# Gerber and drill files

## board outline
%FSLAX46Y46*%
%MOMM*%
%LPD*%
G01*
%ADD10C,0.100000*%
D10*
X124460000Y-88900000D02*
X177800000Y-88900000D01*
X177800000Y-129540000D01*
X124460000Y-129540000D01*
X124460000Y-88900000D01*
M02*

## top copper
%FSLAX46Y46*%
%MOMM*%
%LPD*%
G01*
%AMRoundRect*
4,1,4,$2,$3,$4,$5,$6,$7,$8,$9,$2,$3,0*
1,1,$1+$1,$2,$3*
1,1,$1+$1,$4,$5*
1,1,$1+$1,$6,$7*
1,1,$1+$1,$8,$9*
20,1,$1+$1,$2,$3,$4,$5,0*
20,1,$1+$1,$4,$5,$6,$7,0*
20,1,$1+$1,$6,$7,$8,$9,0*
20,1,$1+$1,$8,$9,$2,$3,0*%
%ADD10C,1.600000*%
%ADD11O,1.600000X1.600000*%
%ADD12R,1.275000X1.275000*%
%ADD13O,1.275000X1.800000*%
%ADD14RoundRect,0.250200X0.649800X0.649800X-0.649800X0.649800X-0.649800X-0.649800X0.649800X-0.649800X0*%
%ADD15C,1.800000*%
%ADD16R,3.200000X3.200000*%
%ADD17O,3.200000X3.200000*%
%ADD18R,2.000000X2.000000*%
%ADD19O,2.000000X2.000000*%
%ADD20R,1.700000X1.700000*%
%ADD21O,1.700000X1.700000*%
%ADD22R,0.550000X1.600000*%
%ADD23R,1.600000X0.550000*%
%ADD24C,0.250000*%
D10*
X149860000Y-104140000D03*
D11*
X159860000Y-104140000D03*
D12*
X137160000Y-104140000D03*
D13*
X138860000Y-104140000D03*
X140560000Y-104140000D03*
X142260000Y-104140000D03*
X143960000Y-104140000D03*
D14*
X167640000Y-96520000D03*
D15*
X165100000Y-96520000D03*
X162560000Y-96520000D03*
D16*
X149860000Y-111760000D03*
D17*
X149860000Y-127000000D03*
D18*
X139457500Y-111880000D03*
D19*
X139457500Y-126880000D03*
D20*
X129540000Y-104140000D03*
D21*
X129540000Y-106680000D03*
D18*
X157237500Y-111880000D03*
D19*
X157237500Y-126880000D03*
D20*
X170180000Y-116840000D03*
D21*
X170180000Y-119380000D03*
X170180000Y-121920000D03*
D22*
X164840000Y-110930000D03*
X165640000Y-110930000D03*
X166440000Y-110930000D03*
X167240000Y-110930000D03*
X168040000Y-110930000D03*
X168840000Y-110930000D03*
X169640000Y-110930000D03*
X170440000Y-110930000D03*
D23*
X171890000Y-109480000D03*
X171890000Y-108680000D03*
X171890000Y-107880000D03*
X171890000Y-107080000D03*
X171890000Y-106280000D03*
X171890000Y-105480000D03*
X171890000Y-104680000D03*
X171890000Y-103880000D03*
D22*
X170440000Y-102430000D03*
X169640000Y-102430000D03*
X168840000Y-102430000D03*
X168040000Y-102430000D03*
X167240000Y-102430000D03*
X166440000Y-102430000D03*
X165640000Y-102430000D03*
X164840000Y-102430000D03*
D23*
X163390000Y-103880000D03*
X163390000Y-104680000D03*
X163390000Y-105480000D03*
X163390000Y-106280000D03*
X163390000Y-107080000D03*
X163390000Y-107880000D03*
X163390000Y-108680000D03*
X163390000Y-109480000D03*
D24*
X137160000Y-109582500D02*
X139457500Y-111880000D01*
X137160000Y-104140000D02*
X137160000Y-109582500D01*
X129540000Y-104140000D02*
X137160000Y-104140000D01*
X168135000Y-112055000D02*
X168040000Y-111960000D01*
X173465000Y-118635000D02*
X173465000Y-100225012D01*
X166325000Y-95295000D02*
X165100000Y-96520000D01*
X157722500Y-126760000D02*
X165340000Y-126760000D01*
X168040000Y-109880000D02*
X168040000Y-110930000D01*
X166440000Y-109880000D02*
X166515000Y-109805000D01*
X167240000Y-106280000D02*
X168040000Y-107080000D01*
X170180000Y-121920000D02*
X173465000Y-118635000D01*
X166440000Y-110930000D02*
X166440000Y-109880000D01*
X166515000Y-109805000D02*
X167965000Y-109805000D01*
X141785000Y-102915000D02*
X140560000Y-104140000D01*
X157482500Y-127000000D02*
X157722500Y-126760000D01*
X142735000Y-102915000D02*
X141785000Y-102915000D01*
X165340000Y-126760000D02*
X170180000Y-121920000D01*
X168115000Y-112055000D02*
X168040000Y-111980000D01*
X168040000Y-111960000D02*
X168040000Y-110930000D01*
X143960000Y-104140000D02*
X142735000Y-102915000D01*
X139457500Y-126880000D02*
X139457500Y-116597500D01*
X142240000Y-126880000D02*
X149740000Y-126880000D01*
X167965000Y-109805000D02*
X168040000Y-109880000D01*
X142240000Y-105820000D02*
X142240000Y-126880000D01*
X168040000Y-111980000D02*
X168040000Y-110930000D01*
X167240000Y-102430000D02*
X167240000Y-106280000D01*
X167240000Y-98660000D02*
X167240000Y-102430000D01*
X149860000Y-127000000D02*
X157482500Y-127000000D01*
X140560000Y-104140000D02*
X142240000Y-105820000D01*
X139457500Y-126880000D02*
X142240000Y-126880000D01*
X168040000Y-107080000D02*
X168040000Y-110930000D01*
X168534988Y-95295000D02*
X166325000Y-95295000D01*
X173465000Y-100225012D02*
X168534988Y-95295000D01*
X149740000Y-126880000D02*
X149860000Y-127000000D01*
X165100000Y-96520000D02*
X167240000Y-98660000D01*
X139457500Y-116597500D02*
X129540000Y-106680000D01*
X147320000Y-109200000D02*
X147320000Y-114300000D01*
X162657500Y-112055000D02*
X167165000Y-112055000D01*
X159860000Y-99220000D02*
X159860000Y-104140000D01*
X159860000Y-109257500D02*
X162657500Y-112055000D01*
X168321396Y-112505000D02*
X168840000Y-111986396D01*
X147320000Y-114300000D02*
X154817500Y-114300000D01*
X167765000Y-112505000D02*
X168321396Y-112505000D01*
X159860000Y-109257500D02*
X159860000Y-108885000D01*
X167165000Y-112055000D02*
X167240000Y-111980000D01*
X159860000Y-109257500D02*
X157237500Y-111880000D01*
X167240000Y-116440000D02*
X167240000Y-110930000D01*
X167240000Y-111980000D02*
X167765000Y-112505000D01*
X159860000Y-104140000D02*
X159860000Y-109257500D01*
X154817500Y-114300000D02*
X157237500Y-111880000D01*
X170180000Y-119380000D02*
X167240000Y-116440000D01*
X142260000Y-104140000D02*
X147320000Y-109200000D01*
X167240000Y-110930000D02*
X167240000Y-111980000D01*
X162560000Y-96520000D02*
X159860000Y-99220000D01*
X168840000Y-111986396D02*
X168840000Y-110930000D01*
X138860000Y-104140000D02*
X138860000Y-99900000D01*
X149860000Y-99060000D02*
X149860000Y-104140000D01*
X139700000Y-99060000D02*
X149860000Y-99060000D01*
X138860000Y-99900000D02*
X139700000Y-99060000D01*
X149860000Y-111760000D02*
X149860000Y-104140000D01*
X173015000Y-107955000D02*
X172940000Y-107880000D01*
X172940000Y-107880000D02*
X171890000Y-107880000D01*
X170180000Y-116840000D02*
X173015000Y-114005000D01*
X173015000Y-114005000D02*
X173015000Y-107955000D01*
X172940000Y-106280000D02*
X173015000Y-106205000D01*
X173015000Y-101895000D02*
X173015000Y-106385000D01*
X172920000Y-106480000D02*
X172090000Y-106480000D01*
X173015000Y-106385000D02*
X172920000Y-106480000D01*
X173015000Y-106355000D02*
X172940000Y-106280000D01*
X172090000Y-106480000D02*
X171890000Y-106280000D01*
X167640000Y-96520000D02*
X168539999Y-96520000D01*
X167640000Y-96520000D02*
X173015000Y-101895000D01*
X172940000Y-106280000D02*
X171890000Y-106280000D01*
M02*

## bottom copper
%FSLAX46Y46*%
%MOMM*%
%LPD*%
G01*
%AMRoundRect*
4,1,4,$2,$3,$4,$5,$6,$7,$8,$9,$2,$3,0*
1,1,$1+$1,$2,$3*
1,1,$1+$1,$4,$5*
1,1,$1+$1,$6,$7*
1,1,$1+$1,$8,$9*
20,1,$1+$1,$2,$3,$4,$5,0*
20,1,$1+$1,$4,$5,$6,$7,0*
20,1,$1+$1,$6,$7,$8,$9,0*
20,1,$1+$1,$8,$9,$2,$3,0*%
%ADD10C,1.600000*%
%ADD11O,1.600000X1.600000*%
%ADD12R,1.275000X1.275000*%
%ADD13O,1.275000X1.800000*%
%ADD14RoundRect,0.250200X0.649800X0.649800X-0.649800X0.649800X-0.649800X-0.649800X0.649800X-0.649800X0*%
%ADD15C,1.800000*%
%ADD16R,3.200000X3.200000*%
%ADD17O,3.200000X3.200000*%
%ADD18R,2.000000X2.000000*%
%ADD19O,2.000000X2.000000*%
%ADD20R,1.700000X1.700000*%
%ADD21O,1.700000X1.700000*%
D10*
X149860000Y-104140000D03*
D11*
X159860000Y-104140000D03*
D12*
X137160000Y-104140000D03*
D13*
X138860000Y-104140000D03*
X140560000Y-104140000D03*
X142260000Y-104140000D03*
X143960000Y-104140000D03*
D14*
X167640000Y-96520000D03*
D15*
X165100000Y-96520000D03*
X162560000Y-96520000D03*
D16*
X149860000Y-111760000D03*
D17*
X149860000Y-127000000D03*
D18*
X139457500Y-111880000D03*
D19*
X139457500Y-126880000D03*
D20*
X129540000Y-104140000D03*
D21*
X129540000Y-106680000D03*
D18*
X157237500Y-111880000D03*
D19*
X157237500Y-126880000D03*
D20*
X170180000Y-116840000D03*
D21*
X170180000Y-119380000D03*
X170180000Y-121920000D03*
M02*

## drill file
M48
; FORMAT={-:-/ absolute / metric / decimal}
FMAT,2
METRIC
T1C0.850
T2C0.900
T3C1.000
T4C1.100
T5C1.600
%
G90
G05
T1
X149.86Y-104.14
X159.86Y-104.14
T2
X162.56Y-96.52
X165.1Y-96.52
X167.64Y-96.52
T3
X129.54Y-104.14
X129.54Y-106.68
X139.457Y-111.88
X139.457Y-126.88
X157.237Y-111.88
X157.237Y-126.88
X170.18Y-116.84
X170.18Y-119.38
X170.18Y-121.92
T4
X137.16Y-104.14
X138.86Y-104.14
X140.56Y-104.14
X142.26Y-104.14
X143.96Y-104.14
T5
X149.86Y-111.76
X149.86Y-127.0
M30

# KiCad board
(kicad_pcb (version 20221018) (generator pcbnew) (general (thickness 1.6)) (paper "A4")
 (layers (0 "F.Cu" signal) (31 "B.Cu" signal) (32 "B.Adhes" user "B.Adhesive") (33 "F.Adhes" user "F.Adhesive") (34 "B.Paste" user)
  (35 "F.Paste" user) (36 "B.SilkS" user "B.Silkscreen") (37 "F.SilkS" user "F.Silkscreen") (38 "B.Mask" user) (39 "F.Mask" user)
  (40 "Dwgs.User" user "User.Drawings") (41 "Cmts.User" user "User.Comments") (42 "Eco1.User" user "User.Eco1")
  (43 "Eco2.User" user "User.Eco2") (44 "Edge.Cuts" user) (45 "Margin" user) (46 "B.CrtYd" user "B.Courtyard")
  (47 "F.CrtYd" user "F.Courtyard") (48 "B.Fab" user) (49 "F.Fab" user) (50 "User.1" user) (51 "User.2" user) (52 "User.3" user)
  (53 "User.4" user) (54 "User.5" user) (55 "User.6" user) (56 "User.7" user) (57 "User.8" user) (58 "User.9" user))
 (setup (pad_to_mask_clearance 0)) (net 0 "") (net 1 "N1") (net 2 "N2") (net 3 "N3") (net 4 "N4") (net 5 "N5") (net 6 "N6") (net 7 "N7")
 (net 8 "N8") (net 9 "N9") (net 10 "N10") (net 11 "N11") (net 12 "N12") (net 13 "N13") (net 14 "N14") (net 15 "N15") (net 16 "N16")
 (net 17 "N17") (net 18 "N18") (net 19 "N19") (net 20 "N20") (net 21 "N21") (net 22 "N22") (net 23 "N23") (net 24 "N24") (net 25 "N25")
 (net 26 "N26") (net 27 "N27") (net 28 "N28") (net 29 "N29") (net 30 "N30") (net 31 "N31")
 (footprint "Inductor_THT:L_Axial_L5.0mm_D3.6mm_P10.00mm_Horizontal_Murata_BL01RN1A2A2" (layer "F.Cu") (at 149.86 104.14)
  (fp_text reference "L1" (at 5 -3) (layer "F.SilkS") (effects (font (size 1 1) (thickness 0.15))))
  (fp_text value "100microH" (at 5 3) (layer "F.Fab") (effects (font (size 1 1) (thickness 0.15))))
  (pad "1" thru_hole circle (at 0 0) (size 1.6 1.6) (drill 0.85) (layers "*.Cu" "*.Mask") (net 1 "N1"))
  (pad "2" thru_hole oval (at 10 0) (size 1.6 1.6) (drill 0.85) (layers "*.Cu" "*.Mask") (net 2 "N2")))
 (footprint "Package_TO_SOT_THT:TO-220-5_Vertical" (layer "F.Cu") (at 137.16 104.14)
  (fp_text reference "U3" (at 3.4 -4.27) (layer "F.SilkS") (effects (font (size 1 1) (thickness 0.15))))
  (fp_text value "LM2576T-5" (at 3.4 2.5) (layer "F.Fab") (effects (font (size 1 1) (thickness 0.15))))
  (pad "1" thru_hole rect (at 0 0) (size 1.275 1.275) (drill 1.1) (layers "*.Cu" "*.Mask") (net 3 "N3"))
  (pad "2" thru_hole oval (at 1.7 0) (size 1.275 1.8) (drill 1.1) (layers "*.Cu" "*.Mask") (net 1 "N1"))
  (pad "3" thru_hole oval (at 3.4 0) (size 1.275 1.8) (drill 1.1) (layers "*.Cu" "*.Mask") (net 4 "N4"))
  (pad "4" thru_hole oval (at 5.1 0) (size 1.275 1.8) (drill 1.1) (layers "*.Cu" "*.Mask") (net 2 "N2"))
  (pad "5" thru_hole oval (at 6.8 0) (size 1.275 1.8) (drill 1.1) (layers "*.Cu" "*.Mask") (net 4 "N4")))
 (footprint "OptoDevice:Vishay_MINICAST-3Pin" (layer "F.Cu") (at 167.64 96.52 180)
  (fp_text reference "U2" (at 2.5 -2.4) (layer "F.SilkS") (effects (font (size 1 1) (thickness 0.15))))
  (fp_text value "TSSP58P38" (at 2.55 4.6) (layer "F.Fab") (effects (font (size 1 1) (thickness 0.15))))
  (pad "1" thru_hole roundrect (at 0 0 180) (size 1.8 1.8) (drill 0.9) (layers "*.Cu" "*.Mask") (roundrect_rratio 0.139) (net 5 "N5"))
  (pad "2" thru_hole circle (at 2.54 0 180) (size 1.8 1.8) (drill 0.9) (layers "*.Cu" "*.Mask") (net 4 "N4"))
  (pad "3" thru_hole circle (at 5.08 0 180) (size 1.8 1.8) (drill 0.9) (layers "*.Cu" "*.Mask") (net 2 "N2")))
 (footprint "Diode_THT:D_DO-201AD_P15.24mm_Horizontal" (layer "F.Cu") (at 149.86 111.76 -90)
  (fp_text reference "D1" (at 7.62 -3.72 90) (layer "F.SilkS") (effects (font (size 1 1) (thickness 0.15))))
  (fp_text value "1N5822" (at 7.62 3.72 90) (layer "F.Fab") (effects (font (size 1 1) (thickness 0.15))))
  (pad "1" thru_hole rect (at 0 0 270) (size 3.2 3.2) (drill 1.6) (layers "*.Cu" "*.Mask") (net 1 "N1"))
  (pad "2" thru_hole oval (at 15.24 0 270) (size 3.2 3.2) (drill 1.6) (layers "*.Cu" "*.Mask") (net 4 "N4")))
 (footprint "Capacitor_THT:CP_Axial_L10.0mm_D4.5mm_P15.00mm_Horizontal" (layer "F.Cu") (at 139.4575 111.88 -90)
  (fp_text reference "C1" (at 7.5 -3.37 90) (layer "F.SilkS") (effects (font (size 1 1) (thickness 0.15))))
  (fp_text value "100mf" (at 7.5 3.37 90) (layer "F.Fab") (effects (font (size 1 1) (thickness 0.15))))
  (pad "1" thru_hole rect (at 0 0 270) (size 2 2) (drill 1) (layers "*.Cu" "*.Mask") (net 3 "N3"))
  (pad "2" thru_hole oval (at 15 0 270) (size 2 2) (drill 1) (layers "*.Cu" "*.Mask") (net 4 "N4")))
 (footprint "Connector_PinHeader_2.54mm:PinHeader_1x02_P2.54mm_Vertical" (layer "F.Cu") (at 129.54 104.14)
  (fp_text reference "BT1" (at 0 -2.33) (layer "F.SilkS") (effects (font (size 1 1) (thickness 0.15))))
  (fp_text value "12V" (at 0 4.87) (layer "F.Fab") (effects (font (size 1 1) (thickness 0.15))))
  (pad "1" thru_hole rect (at 0 0) (size 1.7 1.7) (drill 1) (layers "*.Cu" "*.Mask") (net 3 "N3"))
  (pad "2" thru_hole oval (at 0 2.54) (size 1.7 1.7) (drill 1) (layers "*.Cu" "*.Mask") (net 4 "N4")))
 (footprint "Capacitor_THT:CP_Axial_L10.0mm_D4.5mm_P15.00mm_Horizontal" (layer "F.Cu") (at 157.2375 111.88 -90)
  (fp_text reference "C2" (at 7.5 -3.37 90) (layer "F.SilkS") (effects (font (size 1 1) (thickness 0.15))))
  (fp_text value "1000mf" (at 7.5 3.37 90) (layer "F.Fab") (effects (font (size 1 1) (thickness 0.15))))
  (pad "1" thru_hole rect (at 0 0 270) (size 2 2) (drill 1) (layers "*.Cu" "*.Mask") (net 2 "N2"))
  (pad "2" thru_hole oval (at 15 0 270) (size 2 2) (drill 1) (layers "*.Cu" "*.Mask") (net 4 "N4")))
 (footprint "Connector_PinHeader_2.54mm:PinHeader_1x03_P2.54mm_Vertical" (layer "F.Cu") (at 170.18 116.84)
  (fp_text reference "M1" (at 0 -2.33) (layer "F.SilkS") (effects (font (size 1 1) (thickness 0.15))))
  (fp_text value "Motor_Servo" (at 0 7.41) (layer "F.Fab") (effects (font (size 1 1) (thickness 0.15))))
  (pad "1" thru_hole rect (at 0 0) (size 1.7 1.7) (drill 1) (layers "*.Cu" "*.Mask") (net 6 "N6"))
  (pad "2" thru_hole oval (at 0 2.54) (size 1.7 1.7) (drill 1) (layers "*.Cu" "*.Mask") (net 2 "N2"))
  (pad "3" thru_hole oval (at 0 5.08) (size 1.7 1.7) (drill 1) (layers "*.Cu" "*.Mask") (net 4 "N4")))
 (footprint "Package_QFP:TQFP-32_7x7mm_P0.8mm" (layer "F.Cu") (at 167.64 106.68 90)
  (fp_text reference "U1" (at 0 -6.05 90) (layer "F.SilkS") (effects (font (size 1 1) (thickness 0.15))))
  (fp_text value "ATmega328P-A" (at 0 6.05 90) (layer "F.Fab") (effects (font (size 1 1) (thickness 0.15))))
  (pad "1" smd rect (at -4.25 -2.8 90) (size 1.6 0.55) (layers "F.Cu" "F.Paste" "F.Mask") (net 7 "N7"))
  (pad "2" smd rect (at -4.25 -2 90) (size 1.6 0.55) (layers "F.Cu" "F.Paste" "F.Mask") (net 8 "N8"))
  (pad "3" smd rect (at -4.25 -1.2 90) (size 1.6 0.55) (layers "F.Cu" "F.Paste" "F.Mask") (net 4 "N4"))
  (pad "4" smd rect (at -4.25 -0.4 90) (size 1.6 0.55) (layers "F.Cu" "F.Paste" "F.Mask") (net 2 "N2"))
  (pad "5" smd rect (at -4.25 0.4 90) (size 1.6 0.55) (layers "F.Cu" "F.Paste" "F.Mask") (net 4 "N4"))
  (pad "6" smd rect (at -4.25 1.2 90) (size 1.6 0.55) (layers "F.Cu" "F.Paste" "F.Mask") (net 2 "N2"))
  (pad "7" smd rect (at -4.25 2 90) (size 1.6 0.55) (layers "F.Cu" "F.Paste" "F.Mask") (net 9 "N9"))
  (pad "8" smd rect (at -4.25 2.8 90) (size 1.6 0.55) (layers "F.Cu" "F.Paste" "F.Mask") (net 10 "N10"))
  (pad "9" smd rect (at -2.8 4.25 180) (size 1.6 0.55) (layers "F.Cu" "F.Paste" "F.Mask") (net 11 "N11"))
  (pad "10" smd rect (at -2 4.25 180) (size 1.6 0.55) (layers "F.Cu" "F.Paste" "F.Mask") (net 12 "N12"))
  (pad "11" smd rect (at -1.2 4.25 180) (size 1.6 0.55) (layers "F.Cu" "F.Paste" "F.Mask") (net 6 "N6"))
  (pad "12" smd rect (at -0.4 4.25 180) (size 1.6 0.55) (layers "F.Cu" "F.Paste" "F.Mask") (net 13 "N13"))
  (pad "13" smd rect (at 0.4 4.25 180) (size 1.6 0.55) (layers "F.Cu" "F.Paste" "F.Mask") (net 5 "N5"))
  (pad "14" smd rect (at 1.2 4.25 180) (size 1.6 0.55) (layers "F.Cu" "F.Paste" "F.Mask") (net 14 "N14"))
  (pad "15" smd rect (at 2 4.25 180) (size 1.6 0.55) (layers "F.Cu" "F.Paste" "F.Mask") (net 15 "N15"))
  (pad "16" smd rect (at 2.8 4.25 180) (size 1.6 0.55) (layers "F.Cu" "F.Paste" "F.Mask") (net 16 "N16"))
  (pad "17" smd rect (at 4.25 2.8 90) (size 1.6 0.55) (layers "F.Cu" "F.Paste" "F.Mask") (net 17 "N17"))
  (pad "18" smd rect (at 4.25 2 90) (size 1.6 0.55) (layers "F.Cu" "F.Paste" "F.Mask") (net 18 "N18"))
  (pad "19" smd rect (at 4.25 1.2 90) (size 1.6 0.55) (layers "F.Cu" "F.Paste" "F.Mask") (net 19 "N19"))
  (pad "20" smd rect (at 4.25 0.4 90) (size 1.6 0.55) (layers "F.Cu" "F.Paste" "F.Mask") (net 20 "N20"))
  (pad "21" smd rect (at 4.25 -0.4 90) (size 1.6 0.55) (layers "F.Cu" "F.Paste" "F.Mask") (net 4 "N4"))
  (pad "22" smd rect (at 4.25 -1.2 90) (size 1.6 0.55) (layers "F.Cu" "F.Paste" "F.Mask") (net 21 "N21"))
  (pad "23" smd rect (at 4.25 -2 90) (size 1.6 0.55) (layers "F.Cu" "F.Paste" "F.Mask") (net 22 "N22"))
  (pad "24" smd rect (at 4.25 -2.8 90) (size 1.6 0.55) (layers "F.Cu" "F.Paste" "F.Mask") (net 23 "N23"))
  (pad "25" smd rect (at 2.8 -4.25 180) (size 1.6 0.55) (layers "F.Cu" "F.Paste" "F.Mask") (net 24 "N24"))
  (pad "26" smd rect (at 2 -4.25 180) (size 1.6 0.55) (layers "F.Cu" "F.Paste" "F.Mask") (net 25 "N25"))
  (pad "27" smd rect (at 1.2 -4.25 180) (size 1.6 0.55) (layers "F.Cu" "F.Paste" "F.Mask") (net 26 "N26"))
  (pad "28" smd rect (at 0.4 -4.25 180) (size 1.6 0.55) (layers "F.Cu" "F.Paste" "F.Mask") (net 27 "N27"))
  (pad "29" smd rect (at -0.4 -4.25 180) (size 1.6 0.55) (layers "F.Cu" "F.Paste" "F.Mask") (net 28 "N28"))
  (pad "30" smd rect (at -1.2 -4.25 180) (size 1.6 0.55) (layers "F.Cu" "F.Paste" "F.Mask") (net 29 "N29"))
  (pad "31" smd rect (at -2 -4.25 180) (size 1.6 0.55) (layers "F.Cu" "F.Paste" "F.Mask") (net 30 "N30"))
  (pad "32" smd rect (at -2.8 -4.25 180) (size 1.6 0.55) (layers "F.Cu" "F.Paste" "F.Mask") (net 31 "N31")))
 (gr_rect (start 124.46 88.9) (end 177.8 129.54) (stroke (width 0.1) (type default)) (fill none) (layer "Edge.Cuts"))
 (segment (start 137.16 109.5825) (end 139.4575 111.88) (width 0.25) (layer "F.Cu") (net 3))
 (segment (start 137.16 104.14) (end 137.16 109.5825) (width 0.25) (layer "F.Cu") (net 3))
 (segment (start 129.54 104.14) (end 137.16 104.14) (width 0.25) (layer "F.Cu") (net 3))
 (segment (start 168.135 112.055) (end 168.04 111.96) (width 0.25) (layer "F.Cu") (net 4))
 (segment (start 173.465 118.635) (end 173.465 100.225012) (width 0.25) (layer "F.Cu") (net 4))
 (segment (start 166.325 95.295) (end 165.1 96.52) (width 0.25) (layer "F.Cu") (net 4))
 (segment (start 157.7225 126.76) (end 165.34 126.76) (width 0.25) (layer "F.Cu") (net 4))
 (segment (start 168.04 109.88) (end 168.04 110.93) (width 0.25) (layer "F.Cu") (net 4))
 (segment (start 166.44 109.88) (end 166.515 109.805) (width 0.25) (layer "F.Cu") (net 4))
 (segment (start 167.24 106.28) (end 168.04 107.08) (width 0.25) (layer "F.Cu") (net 4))
 (segment (start 170.18 121.92) (end 173.465 118.635) (width 0.25) (layer "F.Cu") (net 4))
 (segment (start 166.44 110.93) (end 166.44 109.88) (width 0.25) (layer "F.Cu") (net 4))
 (segment (start 166.515 109.805) (end 167.965 109.805) (width 0.25) (layer "F.Cu") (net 4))
 (segment (start 141.785 102.915) (end 140.56 104.14) (width 0.25) (layer "F.Cu") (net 4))
 (segment (start 157.4825 127) (end 157.7225 126.76) (width 0.25) (layer "F.Cu") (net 4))
 (segment (start 142.735 102.915) (end 141.785 102.915) (width 0.25) (layer "F.Cu") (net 4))
 (segment (start 165.34 126.76) (end 170.18 121.92) (width 0.25) (layer "F.Cu") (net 4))
 (segment (start 168.115 112.055) (end 168.04 111.98) (width 0.25) (layer "F.Cu") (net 4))
 (segment (start 168.04 111.96) (end 168.04 110.93) (width 0.25) (layer "F.Cu") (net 4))
 (segment (start 143.96 104.14) (end 142.735 102.915) (width 0.25) (layer "F.Cu") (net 4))
 (segment (start 139.4575 126.88) (end 139.4575 116.5975) (width 0.25) (layer "F.Cu") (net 4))
 (segment (start 142.24 126.88) (end 149.74 126.88) (width 0.25) (layer "F.Cu") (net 4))
 (segment (start 167.965 109.805) (end 168.04 109.88) (width 0.25) (layer "F.Cu") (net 4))
 (segment (start 142.24 105.82) (end 142.24 126.88) (width 0.25) (layer "F.Cu") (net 4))
 (segment (start 168.04 111.98) (end 168.04 110.93) (width 0.25) (layer "F.Cu") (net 4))
 (segment (start 167.24 102.43) (end 167.24 106.28) (width 0.25) (layer "F.Cu") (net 4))
 (segment (start 167.24 98.66) (end 167.24 102.43) (width 0.25) (layer "F.Cu") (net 4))
 (segment (start 149.86 127) (end 157.4825 127) (width 0.25) (layer "F.Cu") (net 4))
 (segment (start 140.56 104.14) (end 142.24 105.82) (width 0.25) (layer "F.Cu") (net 4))
 (segment (start 139.4575 126.88) (end 142.24 126.88) (width 0.25) (layer "F.Cu") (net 4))
 (segment (start 168.04 107.08) (end 168.04 110.93) (width 0.25) (layer "F.Cu") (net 4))
 (segment (start 168.534988 95.295) (end 166.325 95.295) (width 0.25) (layer "F.Cu") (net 4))
 (segment (start 173.465 100.225012) (end 168.534988 95.295) (width 0.25) (layer "F.Cu") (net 4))
 (segment (start 149.74 126.88) (end 149.86 127) (width 0.25) (layer "F.Cu") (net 4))
 (segment (start 165.1 96.52) (end 167.24 98.66) (width 0.25) (layer "F.Cu") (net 4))
 (segment (start 139.4575 116.5975) (end 129.54 106.68) (width 0.25) (layer "F.Cu") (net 4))
 (segment (start 147.32 109.2) (end 147.32 114.3) (width 0.25) (layer "F.Cu") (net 2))
 (segment (start 162.6575 112.055) (end 167.165 112.055) (width 0.25) (layer "F.Cu") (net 2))
 (segment (start 159.86 99.22) (end 159.86 104.14) (width 0.25) (layer "F.Cu") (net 2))
 (segment (start 159.86 109.2575) (end 162.6575 112.055) (width 0.25) (layer "F.Cu") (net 2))
 (segment (start 168.321396 112.505) (end 168.84 111.986396) (width 0.25) (layer "F.Cu") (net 2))
 (segment (start 147.32 114.3) (end 154.8175 114.3) (width 0.25) (layer "F.Cu") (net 2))
 (segment (start 167.765 112.505) (end 168.321396 112.505) (width 0.25) (layer "F.Cu") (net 2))
 (segment (start 159.86 109.2575) (end 159.86 108.885) (width 0.25) (layer "F.Cu") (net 2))
 (segment (start 167.165 112.055) (end 167.24 111.98) (width 0.25) (layer "F.Cu") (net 2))
 (segment (start 159.86 109.2575) (end 157.2375 111.88) (width 0.25) (layer "F.Cu") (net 2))
 (segment (start 167.24 116.44) (end 167.24 110.93) (width 0.25) (layer "F.Cu") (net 2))
 (segment (start 167.24 111.98) (end 167.765 112.505) (width 0.25) (layer "F.Cu") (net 2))
 (segment (start 159.86 104.14) (end 159.86 109.2575) (width 0.25) (layer "F.Cu") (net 2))
 (segment (start 154.8175 114.3) (end 157.2375 111.88) (width 0.25) (layer "F.Cu") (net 2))
 (segment (start 170.18 119.38) (end 167.24 116.44) (width 0.25) (layer "F.Cu") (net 2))
 (segment (start 142.26 104.14) (end 147.32 109.2) (width 0.25) (layer "F.Cu") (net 2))
 (segment (start 167.24 110.93) (end 167.24 111.98) (width 0.25) (layer "F.Cu") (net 2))
 (segment (start 162.56 96.52) (end 159.86 99.22) (width 0.25) (layer "F.Cu") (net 2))
 (segment (start 168.84 111.986396) (end 168.84 110.93) (width 0.25) (layer "F.Cu") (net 2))
 (segment (start 138.86 104.14) (end 138.86 99.9) (width 0.25) (layer "F.Cu") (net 1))
 (segment (start 149.86 99.06) (end 149.86 104.14) (width 0.25) (layer "F.Cu") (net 1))
 (segment (start 139.7 99.06) (end 149.86 99.06) (width 0.25) (layer "F.Cu") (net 1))
 (segment (start 138.86 99.9) (end 139.7 99.06) (width 0.25) (layer "F.Cu") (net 1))
 (segment (start 149.86 111.76) (end 149.86 104.14) (width 0.25) (layer "F.Cu") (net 1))
 (segment (start 173.015 107.955) (end 172.94 107.88) (width 0.25) (layer "F.Cu") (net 6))
 (segment (start 172.94 107.88) (end 171.89 107.88) (width 0.25) (layer "F.Cu") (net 6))
 (segment (start 170.18 116.84) (end 173.015 114.005) (width 0.25) (layer "F.Cu") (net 6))
 (segment (start 173.015 114.005) (end 173.015 107.955) (width 0.25) (layer "F.Cu") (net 6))
 (segment (start 172.94 106.28) (end 173.015 106.205) (width 0.25) (layer "F.Cu") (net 5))
 (segment (start 173.015 101.895) (end 173.015 106.385) (width 0.25) (layer "F.Cu") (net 5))
 (segment (start 172.92 106.48) (end 172.09 106.48) (width 0.25) (layer "F.Cu") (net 5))
 (segment (start 173.015 106.385) (end 172.92 106.48) (width 0.25) (layer "F.Cu") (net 5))
 (segment (start 173.015 106.355) (end 172.94 106.28) (width 0.25) (layer "F.Cu") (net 5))
 (segment (start 172.09 106.48) (end 171.89 106.28) (width 0.25) (layer "F.Cu") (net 5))
 (segment (start 167.64 96.52) (end 168.539999 96.52) (width 0.25) (layer "F.Cu") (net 5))
 (segment (start 167.64 96.52) (end 173.015 101.895) (width 0.25) (layer "F.Cu") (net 5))
 (segment (start 172.94 106.28) (end 171.89 106.28) (width 0.25) (layer "F.Cu") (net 5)))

